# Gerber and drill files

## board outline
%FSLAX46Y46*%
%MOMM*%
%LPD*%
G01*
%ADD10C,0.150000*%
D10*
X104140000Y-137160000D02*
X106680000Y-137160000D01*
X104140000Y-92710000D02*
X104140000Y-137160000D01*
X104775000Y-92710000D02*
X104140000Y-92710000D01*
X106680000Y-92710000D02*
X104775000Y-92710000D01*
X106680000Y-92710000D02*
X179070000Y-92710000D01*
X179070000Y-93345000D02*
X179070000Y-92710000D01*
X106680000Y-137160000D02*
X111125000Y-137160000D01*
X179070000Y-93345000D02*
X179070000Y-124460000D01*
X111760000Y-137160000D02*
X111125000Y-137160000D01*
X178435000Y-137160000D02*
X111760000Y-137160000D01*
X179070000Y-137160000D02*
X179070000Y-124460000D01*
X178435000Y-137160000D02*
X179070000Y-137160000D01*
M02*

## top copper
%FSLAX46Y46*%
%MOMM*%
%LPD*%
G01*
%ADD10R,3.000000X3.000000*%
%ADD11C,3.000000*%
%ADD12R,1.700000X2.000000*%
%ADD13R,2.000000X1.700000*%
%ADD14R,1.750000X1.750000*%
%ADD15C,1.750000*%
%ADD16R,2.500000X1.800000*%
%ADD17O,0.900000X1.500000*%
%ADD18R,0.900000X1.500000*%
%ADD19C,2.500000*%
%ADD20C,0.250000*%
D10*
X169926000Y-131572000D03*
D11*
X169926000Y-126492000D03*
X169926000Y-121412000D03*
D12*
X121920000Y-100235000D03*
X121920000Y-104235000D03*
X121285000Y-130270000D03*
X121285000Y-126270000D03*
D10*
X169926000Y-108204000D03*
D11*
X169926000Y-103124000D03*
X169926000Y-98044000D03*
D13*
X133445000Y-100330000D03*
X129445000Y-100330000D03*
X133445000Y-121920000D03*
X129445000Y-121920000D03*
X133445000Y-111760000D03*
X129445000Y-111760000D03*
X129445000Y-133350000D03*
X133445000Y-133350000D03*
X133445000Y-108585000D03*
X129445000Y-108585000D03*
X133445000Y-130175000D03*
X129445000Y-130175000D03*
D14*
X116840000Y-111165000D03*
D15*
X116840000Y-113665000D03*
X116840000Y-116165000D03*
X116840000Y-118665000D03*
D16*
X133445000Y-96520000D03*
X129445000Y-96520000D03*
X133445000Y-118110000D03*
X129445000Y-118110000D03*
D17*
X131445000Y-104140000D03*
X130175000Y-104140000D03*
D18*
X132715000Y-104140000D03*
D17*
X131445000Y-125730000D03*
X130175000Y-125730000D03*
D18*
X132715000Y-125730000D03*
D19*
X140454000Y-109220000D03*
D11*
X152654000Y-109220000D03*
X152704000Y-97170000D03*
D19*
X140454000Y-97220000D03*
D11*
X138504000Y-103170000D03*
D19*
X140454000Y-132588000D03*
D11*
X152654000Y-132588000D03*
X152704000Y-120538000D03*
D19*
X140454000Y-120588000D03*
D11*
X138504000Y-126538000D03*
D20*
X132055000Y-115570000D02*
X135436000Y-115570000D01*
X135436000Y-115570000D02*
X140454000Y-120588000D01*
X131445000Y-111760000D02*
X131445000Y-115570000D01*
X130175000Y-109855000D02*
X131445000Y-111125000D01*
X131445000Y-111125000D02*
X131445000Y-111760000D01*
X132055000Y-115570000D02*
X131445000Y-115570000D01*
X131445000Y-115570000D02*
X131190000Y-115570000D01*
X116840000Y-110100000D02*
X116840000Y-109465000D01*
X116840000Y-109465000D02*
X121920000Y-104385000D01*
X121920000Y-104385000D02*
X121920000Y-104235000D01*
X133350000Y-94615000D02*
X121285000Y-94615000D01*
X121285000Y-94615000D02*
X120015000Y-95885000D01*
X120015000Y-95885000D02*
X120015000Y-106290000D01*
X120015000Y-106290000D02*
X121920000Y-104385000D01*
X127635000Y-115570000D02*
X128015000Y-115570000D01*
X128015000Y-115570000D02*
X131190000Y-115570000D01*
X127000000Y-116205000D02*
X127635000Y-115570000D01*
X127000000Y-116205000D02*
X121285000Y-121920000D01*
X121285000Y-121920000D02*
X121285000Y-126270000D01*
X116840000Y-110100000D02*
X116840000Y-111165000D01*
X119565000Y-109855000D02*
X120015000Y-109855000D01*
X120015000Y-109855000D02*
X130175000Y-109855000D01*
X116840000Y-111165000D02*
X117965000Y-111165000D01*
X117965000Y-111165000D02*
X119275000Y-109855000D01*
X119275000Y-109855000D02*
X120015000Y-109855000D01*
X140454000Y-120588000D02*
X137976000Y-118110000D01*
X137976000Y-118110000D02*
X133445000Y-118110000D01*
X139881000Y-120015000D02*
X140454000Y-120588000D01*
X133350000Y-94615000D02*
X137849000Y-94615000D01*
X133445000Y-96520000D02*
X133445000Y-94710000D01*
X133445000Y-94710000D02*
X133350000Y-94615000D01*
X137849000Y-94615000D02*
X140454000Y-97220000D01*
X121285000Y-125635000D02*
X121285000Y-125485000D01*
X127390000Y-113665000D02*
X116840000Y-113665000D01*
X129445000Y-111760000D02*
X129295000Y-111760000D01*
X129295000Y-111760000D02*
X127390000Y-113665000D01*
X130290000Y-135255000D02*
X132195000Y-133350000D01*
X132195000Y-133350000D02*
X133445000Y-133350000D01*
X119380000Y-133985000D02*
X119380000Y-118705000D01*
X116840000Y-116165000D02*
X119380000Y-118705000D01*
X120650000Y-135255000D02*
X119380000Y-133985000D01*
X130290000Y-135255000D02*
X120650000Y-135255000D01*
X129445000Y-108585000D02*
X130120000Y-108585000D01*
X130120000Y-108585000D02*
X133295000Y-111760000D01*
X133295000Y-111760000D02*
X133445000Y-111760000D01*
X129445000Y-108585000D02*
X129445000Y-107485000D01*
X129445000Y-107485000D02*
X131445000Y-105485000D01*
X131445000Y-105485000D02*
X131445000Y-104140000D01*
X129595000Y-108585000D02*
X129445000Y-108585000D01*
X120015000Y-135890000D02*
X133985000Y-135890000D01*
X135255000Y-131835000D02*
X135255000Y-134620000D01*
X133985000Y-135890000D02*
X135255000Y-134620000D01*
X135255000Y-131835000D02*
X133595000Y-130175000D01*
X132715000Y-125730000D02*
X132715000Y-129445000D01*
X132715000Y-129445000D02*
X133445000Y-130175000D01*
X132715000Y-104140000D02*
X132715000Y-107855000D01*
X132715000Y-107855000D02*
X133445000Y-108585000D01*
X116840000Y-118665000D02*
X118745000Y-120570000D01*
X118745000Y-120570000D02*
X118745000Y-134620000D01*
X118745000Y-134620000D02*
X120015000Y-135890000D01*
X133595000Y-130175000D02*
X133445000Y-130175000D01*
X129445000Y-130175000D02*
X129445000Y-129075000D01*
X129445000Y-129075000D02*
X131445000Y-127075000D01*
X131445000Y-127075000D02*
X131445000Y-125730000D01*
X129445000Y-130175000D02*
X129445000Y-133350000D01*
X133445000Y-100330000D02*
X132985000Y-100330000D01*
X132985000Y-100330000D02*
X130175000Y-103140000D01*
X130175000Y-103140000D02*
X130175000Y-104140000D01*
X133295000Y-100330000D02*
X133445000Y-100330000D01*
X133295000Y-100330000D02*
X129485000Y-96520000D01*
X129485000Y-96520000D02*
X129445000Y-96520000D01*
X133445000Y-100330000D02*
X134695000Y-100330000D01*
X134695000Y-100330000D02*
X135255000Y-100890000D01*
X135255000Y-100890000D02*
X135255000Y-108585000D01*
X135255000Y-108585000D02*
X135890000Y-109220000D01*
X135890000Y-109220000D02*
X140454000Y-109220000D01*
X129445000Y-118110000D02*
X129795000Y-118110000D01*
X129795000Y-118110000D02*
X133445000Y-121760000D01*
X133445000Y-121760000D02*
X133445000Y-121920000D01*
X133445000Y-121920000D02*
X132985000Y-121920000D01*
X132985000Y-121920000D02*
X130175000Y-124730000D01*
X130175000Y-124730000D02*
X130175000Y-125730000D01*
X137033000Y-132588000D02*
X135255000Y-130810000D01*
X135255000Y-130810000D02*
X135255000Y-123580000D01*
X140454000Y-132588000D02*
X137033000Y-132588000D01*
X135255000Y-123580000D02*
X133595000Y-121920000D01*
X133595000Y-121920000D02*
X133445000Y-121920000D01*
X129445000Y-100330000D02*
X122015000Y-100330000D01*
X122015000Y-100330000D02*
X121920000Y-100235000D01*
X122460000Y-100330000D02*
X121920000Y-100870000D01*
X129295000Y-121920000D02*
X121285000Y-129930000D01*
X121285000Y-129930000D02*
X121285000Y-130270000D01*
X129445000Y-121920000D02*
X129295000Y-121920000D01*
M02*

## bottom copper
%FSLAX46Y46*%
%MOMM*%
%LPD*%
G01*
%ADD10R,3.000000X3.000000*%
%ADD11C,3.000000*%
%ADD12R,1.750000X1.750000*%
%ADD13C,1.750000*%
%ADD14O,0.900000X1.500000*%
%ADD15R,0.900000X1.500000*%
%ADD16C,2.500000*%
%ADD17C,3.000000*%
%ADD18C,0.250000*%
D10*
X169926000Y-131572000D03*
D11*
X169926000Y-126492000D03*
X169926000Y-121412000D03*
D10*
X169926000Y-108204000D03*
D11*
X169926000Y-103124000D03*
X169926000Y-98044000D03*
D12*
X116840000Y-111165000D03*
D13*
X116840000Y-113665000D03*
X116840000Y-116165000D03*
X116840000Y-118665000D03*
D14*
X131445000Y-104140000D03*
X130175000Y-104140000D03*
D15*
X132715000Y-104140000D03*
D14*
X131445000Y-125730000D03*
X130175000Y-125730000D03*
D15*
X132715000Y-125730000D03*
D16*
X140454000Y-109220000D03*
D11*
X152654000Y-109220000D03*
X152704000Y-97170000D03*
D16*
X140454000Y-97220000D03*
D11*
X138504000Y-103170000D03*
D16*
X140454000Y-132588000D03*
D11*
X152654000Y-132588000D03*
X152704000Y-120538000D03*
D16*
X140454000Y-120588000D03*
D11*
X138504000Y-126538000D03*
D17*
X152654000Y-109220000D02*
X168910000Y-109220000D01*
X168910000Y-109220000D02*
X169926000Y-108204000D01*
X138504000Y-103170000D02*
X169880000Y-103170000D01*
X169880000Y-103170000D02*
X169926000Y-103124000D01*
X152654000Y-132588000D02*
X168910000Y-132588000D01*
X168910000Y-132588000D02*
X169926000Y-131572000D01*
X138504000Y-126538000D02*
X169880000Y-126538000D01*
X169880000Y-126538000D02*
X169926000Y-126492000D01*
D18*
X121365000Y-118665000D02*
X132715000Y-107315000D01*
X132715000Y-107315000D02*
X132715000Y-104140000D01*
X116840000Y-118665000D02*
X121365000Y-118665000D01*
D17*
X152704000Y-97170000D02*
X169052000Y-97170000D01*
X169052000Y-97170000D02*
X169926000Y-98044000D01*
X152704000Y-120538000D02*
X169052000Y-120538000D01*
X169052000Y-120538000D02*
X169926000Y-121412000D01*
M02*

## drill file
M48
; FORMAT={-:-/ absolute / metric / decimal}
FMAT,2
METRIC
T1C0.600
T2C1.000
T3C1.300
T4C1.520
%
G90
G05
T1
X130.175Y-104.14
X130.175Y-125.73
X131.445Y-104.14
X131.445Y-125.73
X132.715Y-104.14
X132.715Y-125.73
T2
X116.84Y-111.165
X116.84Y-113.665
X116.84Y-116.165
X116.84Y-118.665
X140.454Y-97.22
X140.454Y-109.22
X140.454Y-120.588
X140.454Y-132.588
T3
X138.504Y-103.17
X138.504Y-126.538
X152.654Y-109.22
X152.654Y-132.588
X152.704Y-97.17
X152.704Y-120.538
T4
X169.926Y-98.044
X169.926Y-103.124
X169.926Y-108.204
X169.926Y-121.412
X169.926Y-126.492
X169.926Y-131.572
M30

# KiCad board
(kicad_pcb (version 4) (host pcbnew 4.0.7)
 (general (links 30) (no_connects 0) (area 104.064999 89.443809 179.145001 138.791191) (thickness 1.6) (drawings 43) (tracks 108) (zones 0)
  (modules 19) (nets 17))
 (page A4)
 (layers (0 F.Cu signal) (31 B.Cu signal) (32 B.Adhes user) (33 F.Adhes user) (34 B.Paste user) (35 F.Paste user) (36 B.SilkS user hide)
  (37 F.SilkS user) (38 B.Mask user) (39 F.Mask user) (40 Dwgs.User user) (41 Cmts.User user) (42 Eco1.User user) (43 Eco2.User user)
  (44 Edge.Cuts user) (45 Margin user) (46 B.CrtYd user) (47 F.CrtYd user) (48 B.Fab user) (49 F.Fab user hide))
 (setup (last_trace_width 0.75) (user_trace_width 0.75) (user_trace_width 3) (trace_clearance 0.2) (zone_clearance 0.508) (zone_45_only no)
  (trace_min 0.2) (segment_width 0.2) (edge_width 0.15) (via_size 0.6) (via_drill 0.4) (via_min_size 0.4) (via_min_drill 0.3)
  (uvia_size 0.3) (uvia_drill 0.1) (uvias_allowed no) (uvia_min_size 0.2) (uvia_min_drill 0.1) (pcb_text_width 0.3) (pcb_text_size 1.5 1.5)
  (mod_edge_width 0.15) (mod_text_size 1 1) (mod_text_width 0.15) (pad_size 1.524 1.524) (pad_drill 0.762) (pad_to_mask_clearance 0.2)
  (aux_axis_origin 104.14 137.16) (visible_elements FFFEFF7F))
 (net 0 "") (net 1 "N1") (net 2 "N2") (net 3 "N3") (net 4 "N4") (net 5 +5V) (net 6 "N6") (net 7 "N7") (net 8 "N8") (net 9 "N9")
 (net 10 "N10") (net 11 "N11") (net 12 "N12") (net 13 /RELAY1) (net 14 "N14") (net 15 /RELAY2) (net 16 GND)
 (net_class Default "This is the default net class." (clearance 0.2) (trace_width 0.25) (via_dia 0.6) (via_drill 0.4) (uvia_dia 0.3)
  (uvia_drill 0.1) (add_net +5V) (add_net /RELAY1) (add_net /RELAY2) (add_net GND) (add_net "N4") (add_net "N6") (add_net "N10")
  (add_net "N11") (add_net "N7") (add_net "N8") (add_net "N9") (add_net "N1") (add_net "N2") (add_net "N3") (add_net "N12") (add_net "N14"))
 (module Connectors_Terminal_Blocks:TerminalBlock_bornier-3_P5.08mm (layer F.Cu) (at 169.926 131.572 90)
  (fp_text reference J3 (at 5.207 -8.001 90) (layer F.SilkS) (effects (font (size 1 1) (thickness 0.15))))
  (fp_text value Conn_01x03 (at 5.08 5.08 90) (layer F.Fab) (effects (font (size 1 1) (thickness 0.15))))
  (pad 1 thru_hole rect (at 0 0 90) (size 3 3) (drill 1.52) (layers *.Cu *.Mask) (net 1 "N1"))
  (pad 2 thru_hole circle (at 5.08 0 90) (size 3 3) (drill 1.52) (layers *.Cu *.Mask) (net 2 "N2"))
  (pad 3 thru_hole circle (at 10.16 0 90) (size 3 3) (drill 1.52) (layers *.Cu *.Mask) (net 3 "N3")))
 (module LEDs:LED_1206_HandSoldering (layer F.Cu) (at 121.92 102.235 270)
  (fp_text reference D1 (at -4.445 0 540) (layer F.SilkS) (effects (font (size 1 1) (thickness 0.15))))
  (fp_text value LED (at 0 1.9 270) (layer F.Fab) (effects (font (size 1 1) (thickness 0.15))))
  (pad 1 smd rect (at -2 0 270) (size 2 1.7) (layers F.Cu F.Paste F.Mask) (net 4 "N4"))
  (pad 2 smd rect (at 2 0 270) (size 2 1.7) (layers F.Cu F.Paste F.Mask) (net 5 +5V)))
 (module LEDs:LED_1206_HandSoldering (layer F.Cu) (at 121.285 128.27 90)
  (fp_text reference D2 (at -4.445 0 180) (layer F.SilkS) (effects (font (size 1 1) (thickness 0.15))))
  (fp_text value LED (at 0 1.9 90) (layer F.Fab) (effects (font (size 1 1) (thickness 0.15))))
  (pad 1 smd rect (at -2 0 90) (size 2 1.7) (layers F.Cu F.Paste F.Mask) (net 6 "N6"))
  (pad 2 smd rect (at 2 0 90) (size 2 1.7) (layers F.Cu F.Paste F.Mask) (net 5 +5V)))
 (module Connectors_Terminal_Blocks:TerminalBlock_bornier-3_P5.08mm (layer F.Cu) (at 169.926 108.204 90)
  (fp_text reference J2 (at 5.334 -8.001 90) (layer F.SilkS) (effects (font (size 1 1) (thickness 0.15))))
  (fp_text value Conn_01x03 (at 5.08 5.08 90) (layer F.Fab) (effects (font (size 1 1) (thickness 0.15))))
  (pad 1 thru_hole rect (at 0 0 90) (size 3 3) (drill 1.52) (layers *.Cu *.Mask) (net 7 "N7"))
  (pad 2 thru_hole circle (at 5.08 0 90) (size 3 3) (drill 1.52) (layers *.Cu *.Mask) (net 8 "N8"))
  (pad 3 thru_hole circle (at 10.16 0 90) (size 3 3) (drill 1.52) (layers *.Cu *.Mask) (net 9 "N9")))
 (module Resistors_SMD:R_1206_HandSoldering (layer F.Cu) (at 131.445 100.33 180)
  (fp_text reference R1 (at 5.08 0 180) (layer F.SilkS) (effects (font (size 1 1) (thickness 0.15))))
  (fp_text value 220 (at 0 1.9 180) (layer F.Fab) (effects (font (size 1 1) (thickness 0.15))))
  (pad 1 smd rect (at -2 0 180) (size 2 1.7) (layers F.Cu F.Paste F.Mask) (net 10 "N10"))
  (pad 2 smd rect (at 2 0 180) (size 2 1.7) (layers F.Cu F.Paste F.Mask) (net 4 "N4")))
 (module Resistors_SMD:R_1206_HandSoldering (layer F.Cu) (at 131.445 121.92 180)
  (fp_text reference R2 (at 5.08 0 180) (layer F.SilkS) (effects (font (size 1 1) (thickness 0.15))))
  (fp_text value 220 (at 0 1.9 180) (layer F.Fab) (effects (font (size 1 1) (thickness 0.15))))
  (pad 1 smd rect (at -2 0 180) (size 2 1.7) (layers F.Cu F.Paste F.Mask) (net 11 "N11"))
  (pad 2 smd rect (at 2 0 180) (size 2 1.7) (layers F.Cu F.Paste F.Mask) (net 6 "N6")))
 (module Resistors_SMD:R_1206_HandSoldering (layer F.Cu) (at 131.445 111.76 180)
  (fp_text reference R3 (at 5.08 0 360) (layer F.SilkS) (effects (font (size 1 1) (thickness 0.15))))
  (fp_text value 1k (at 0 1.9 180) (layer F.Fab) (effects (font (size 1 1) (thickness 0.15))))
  (pad 1 smd rect (at -2 0 180) (size 2 1.7) (layers F.Cu F.Paste F.Mask) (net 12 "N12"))
  (pad 2 smd rect (at 2 0 180) (size 2 1.7) (layers F.Cu F.Paste F.Mask) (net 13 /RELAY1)))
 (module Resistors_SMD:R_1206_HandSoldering (layer F.Cu) (at 131.445 133.35)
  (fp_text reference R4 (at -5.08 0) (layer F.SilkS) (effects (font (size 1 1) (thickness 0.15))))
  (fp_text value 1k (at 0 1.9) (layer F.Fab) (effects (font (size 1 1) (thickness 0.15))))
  (pad 1 smd rect (at -2 0) (size 2 1.7) (layers F.Cu F.Paste F.Mask) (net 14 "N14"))
  (pad 2 smd rect (at 2 0) (size 2 1.7) (layers F.Cu F.Paste F.Mask) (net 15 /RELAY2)))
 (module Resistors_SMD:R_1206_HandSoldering (layer F.Cu) (at 131.445 108.585 180)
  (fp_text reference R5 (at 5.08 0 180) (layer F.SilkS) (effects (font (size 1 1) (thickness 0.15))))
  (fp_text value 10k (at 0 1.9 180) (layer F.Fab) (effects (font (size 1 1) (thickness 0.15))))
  (pad 1 smd rect (at -2 0 180) (size 2 1.7) (layers F.Cu F.Paste F.Mask) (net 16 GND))
  (pad 2 smd rect (at 2 0 180) (size 2 1.7) (layers F.Cu F.Paste F.Mask) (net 12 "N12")))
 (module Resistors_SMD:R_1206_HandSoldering (layer F.Cu) (at 131.445 130.175 180)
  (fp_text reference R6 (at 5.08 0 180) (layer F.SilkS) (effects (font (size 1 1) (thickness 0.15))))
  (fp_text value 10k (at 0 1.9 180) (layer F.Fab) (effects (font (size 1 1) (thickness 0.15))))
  (pad 1 smd rect (at -2 0 180) (size 2 1.7) (layers F.Cu F.Paste F.Mask) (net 16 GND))
  (pad 2 smd rect (at 2 0 180) (size 2 1.7) (layers F.Cu F.Paste F.Mask) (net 14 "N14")))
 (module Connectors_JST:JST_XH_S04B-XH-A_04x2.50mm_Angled (layer F.Cu) (at 116.84 111.165 270)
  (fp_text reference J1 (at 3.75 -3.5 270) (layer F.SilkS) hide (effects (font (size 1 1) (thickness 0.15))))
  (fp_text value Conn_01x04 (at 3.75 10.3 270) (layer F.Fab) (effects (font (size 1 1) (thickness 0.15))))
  (pad 1 thru_hole rect (at 0 0 270) (size 1.75 1.75) (drill 1) (layers *.Cu *.Mask F.SilkS) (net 5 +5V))
  (pad 2 thru_hole circle (at 2.5 0 270) (size 1.75 1.75) (drill 1) (layers *.Cu *.Mask F.SilkS) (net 13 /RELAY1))
  (pad 3 thru_hole circle (at 5 0 270) (size 1.75 1.75) (drill 1) (layers *.Cu *.Mask F.SilkS) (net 15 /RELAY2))
  (pad 4 thru_hole circle (at 7.5 0 270) (size 1.75 1.75) (drill 1) (layers *.Cu *.Mask F.SilkS) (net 16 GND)))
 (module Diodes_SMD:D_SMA (layer F.Cu) (at 131.445 96.52 180)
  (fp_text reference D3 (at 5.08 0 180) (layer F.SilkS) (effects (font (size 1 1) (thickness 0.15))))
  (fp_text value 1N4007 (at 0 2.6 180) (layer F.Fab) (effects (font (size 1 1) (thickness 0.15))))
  (pad 1 smd rect (at -2 0 180) (size 2.5 1.8) (layers F.Cu F.Paste F.Mask) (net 5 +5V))
  (pad 2 smd rect (at 2 0 180) (size 2.5 1.8) (layers F.Cu F.Paste F.Mask) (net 10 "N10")))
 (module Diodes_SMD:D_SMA (layer F.Cu) (at 131.445 118.11 180)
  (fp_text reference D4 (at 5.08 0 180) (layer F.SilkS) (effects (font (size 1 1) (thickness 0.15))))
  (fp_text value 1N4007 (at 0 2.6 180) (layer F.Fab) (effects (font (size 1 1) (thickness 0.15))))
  (pad 1 smd rect (at -2 0 180) (size 2.5 1.8) (layers F.Cu F.Paste F.Mask) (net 5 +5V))
  (pad 2 smd rect (at 2 0 180) (size 2.5 1.8) (layers F.Cu F.Paste F.Mask) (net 11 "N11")))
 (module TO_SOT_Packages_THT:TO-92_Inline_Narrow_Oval (layer F.Cu) (at 132.715 104.14 180)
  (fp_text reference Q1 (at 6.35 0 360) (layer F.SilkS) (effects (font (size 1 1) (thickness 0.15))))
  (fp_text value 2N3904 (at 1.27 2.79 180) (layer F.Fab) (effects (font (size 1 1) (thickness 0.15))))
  (pad 2 thru_hole oval (at 1.27 0) (size 0.9 1.5) (drill 0.6) (layers *.Cu *.Mask) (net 12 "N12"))
  (pad 3 thru_hole oval (at 2.54 0) (size 0.9 1.5) (drill 0.6) (layers *.Cu *.Mask) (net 10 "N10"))
  (pad 1 thru_hole rect (at 0 0) (size 0.9 1.5) (drill 0.6) (layers *.Cu *.Mask) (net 16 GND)))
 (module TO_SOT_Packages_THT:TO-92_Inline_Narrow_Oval (layer F.Cu) (at 132.715 125.73 180)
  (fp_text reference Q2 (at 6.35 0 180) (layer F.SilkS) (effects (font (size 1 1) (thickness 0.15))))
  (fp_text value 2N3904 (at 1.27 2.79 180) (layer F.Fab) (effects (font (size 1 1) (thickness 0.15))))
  (pad 2 thru_hole oval (at 1.27 0) (size 0.9 1.5) (drill 0.6) (layers *.Cu *.Mask) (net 14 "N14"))
  (pad 3 thru_hole oval (at 2.54 0) (size 0.9 1.5) (drill 0.6) (layers *.Cu *.Mask) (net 11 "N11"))
  (pad 1 thru_hole rect (at 0 0) (size 0.9 1.5) (drill 0.6) (layers *.Cu *.Mask) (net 16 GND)))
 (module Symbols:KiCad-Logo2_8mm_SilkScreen (layer B.Cu) (at 161.29 126.365 270)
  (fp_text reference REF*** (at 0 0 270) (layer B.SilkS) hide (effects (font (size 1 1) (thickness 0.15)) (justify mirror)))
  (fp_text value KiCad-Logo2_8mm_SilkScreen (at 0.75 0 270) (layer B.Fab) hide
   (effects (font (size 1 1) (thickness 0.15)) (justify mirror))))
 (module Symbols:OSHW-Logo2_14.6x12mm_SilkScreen (layer B.Cu) (at 160.655 102.87 270)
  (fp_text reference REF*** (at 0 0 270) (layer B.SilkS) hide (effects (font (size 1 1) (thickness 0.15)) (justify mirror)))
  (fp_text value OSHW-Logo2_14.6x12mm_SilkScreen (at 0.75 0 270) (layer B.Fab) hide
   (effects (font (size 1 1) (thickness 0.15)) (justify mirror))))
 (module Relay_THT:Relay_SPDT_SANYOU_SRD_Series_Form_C (layer F.Cu) (at 138.504 103.17)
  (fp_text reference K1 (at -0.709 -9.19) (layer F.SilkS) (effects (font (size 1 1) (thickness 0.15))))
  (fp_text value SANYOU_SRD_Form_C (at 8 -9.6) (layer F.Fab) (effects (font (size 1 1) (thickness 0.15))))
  (pad 2 thru_hole circle (at 1.95 6.05 90) (size 2.5 2.5) (drill 1) (layers *.Cu *.Mask) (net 10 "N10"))
  (pad 3 thru_hole circle (at 14.15 6.05 90) (size 3 3) (drill 1.3) (layers *.Cu *.Mask) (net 7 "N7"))
  (pad 4 thru_hole circle (at 14.2 -6 90) (size 3 3) (drill 1.3) (layers *.Cu *.Mask) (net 9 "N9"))
  (pad 5 thru_hole circle (at 1.95 -5.95 90) (size 2.5 2.5) (drill 1) (layers *.Cu *.Mask) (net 5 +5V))
  (pad 1 thru_hole circle (at 0 0 90) (size 3 3) (drill 1.3) (layers *.Cu *.Mask) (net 8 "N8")))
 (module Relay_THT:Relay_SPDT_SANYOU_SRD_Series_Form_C (layer F.Cu) (at 138.504 126.538)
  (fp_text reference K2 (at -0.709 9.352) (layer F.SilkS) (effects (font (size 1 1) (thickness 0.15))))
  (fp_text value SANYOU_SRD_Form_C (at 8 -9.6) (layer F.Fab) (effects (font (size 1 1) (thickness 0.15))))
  (pad 2 thru_hole circle (at 1.95 6.05 90) (size 2.5 2.5) (drill 1) (layers *.Cu *.Mask) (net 11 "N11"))
  (pad 3 thru_hole circle (at 14.15 6.05 90) (size 3 3) (drill 1.3) (layers *.Cu *.Mask) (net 1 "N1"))
  (pad 4 thru_hole circle (at 14.2 -6 90) (size 3 3) (drill 1.3) (layers *.Cu *.Mask) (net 3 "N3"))
  (pad 5 thru_hole circle (at 1.95 -5.95 90) (size 2.5 2.5) (drill 1) (layers *.Cu *.Mask) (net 5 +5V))
  (pad 1 thru_hole circle (at 0 0 90) (size 3 3) (drill 1.3) (layers *.Cu *.Mask) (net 2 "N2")))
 (gr_line (start 104.14 137.16) (end 106.68 137.16) (layer Edge.Cuts) (width 0.15))
 (gr_line (start 104.14 92.71) (end 104.14 137.16) (layer Edge.Cuts) (width 0.15))
 (gr_line (start 104.775 92.71) (end 104.14 92.71) (layer Edge.Cuts) (width 0.15))
 (gr_line (start 106.68 92.71) (end 104.775 92.71) (layer Edge.Cuts) (width 0.15))
 (gr_line (start 106.68 92.71) (end 179.07 92.71) (layer Edge.Cuts) (width 0.15))
 (gr_line (start 179.07 93.345) (end 179.07 92.71) (layer Edge.Cuts) (width 0.15))
 (gr_line (start 106.68 137.16) (end 111.125 137.16) (layer Edge.Cuts) (width 0.15))
 (gr_line (start 179.07 93.345) (end 179.07 124.46) (layer Edge.Cuts) (width 0.15))
 (gr_line (start 111.76 137.16) (end 111.125 137.16) (layer Edge.Cuts) (width 0.15))
 (gr_line (start 178.435 137.16) (end 111.76 137.16) (layer Edge.Cuts) (width 0.15))
 (gr_line (start 179.07 137.16) (end 179.07 124.46) (layer Edge.Cuts) (width 0.15))
 (gr_line (start 178.435 137.16) (end 179.07 137.16) (layer Edge.Cuts) (width 0.15))
 (segment (start 132.055 115.57) (end 135.436 115.57) (width 0.25) (layer F.Cu) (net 5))
 (segment (start 135.436 115.57) (end 140.454 120.588) (width 0.25) (layer F.Cu) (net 5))
 (segment (start 131.445 111.76) (end 131.445 115.57) (width 0.25) (layer F.Cu) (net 5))
 (segment (start 130.175 109.855) (end 131.445 111.125) (width 0.25) (layer F.Cu) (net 5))
 (segment (start 131.445 111.125) (end 131.445 111.76) (width 0.25) (layer F.Cu) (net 5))
 (segment (start 132.055 115.57) (end 131.445 115.57) (width 0.25) (layer F.Cu) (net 5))
 (segment (start 131.445 115.57) (end 131.19 115.57) (width 0.25) (layer F.Cu) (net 5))
 (segment (start 116.84 110.1) (end 116.84 109.465) (width 0.25) (layer F.Cu) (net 5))
 (segment (start 116.84 109.465) (end 121.92 104.385) (width 0.25) (layer F.Cu) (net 5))
 (segment (start 121.92 104.385) (end 121.92 104.235) (width 0.25) (layer F.Cu) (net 5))
 (segment (start 133.35 94.615) (end 121.285 94.615) (width 0.25) (layer F.Cu) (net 5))
 (segment (start 121.285 94.615) (end 120.015 95.885) (width 0.25) (layer F.Cu) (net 5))
 (segment (start 120.015 95.885) (end 120.015 106.29) (width 0.25) (layer F.Cu) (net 5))
 (segment (start 120.015 106.29) (end 121.92 104.385) (width 0.25) (layer F.Cu) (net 5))
 (segment (start 127.635 115.57) (end 128.015 115.57) (width 0.25) (layer F.Cu) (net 5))
 (segment (start 128.015 115.57) (end 131.19 115.57) (width 0.25) (layer F.Cu) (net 5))
 (segment (start 127 116.205) (end 127.635 115.57) (width 0.25) (layer F.Cu) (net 5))
 (segment (start 127 116.205) (end 121.285 121.92) (width 0.25) (layer F.Cu) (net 5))
 (segment (start 121.285 121.92) (end 121.285 126.27) (width 0.25) (layer F.Cu) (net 5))
 (segment (start 116.84 110.1) (end 116.84 111.165) (width 0.25) (layer F.Cu) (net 5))
 (segment (start 119.565 109.855) (end 120.015 109.855) (width 0.25) (layer F.Cu) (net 5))
 (segment (start 120.015 109.855) (end 130.175 109.855) (width 0.25) (layer F.Cu) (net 5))
 (segment (start 116.84 111.165) (end 117.965 111.165) (width 0.25) (layer F.Cu) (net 5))
 (segment (start 117.965 111.165) (end 119.275 109.855) (width 0.25) (layer F.Cu) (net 5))
 (segment (start 119.275 109.855) (end 120.015 109.855) (width 0.25) (layer F.Cu) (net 5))
 (segment (start 140.454 120.588) (end 137.976 118.11) (width 0.25) (layer F.Cu) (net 5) (status 10))
 (segment (start 137.976 118.11) (end 133.445 118.11) (width 0.25) (layer F.Cu) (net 5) (status 20))
 (segment (start 139.881 120.015) (end 140.454 120.588) (width 0.25) (layer F.Cu) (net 5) (status 30))
 (segment (start 133.35 94.615) (end 137.849 94.615) (width 0.25) (layer F.Cu) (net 5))
 (segment (start 133.445 96.52) (end 133.445 94.71) (width 0.25) (layer F.Cu) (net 5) (status 10))
 (segment (start 133.445 94.71) (end 133.35 94.615) (width 0.25) (layer F.Cu) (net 5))
 (segment (start 137.849 94.615) (end 140.454 97.22) (width 0.25) (layer F.Cu) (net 5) (status 20))
 (segment (start 121.285 125.635) (end 121.285 125.485) (width 0.25) (layer F.Cu) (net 5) (status 30))
 (segment (start 127.39 113.665) (end 116.84 113.665) (width 0.25) (layer F.Cu) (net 13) (status 20))
 (segment (start 129.445 111.76) (end 129.295 111.76) (width 0.25) (layer F.Cu) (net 13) (status 30))
 (segment (start 129.295 111.76) (end 127.39 113.665) (width 0.25) (layer F.Cu) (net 13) (status 10))
 (segment (start 130.29 135.255) (end 132.195 133.35) (width 0.25) (layer F.Cu) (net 15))
 (segment (start 132.195 133.35) (end 133.445 133.35) (width 0.25) (layer F.Cu) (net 15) (status 20))
 (segment (start 119.38 133.985) (end 119.38 118.705) (width 0.25) (layer F.Cu) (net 15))
 (segment (start 116.84 116.165) (end 119.38 118.705) (width 0.25) (layer F.Cu) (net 15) (status 10))
 (segment (start 120.65 135.255) (end 119.38 133.985) (width 0.25) (layer F.Cu) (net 15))
 (segment (start 130.29 135.255) (end 120.65 135.255) (width 0.25) (layer F.Cu) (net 15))
 (segment (start 152.654 109.22) (end 168.91 109.22) (width 3) (layer B.Cu) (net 7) (status 30))
 (segment (start 168.91 109.22) (end 169.926 108.204) (width 3) (layer B.Cu) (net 7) (status 30))
 (segment (start 138.504 103.17) (end 169.88 103.17) (width 3) (layer B.Cu) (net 8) (status 30))
 (segment (start 169.88 103.17) (end 169.926 103.124) (width 3) (layer B.Cu) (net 8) (status 30))
 (segment (start 152.654 132.588) (end 168.91 132.588) (width 3) (layer B.Cu) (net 1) (status 30))
 (segment (start 168.91 132.588) (end 169.926 131.572) (width 3) (layer B.Cu) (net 1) (status 30))
 (segment (start 138.504 126.538) (end 169.88 126.538) (width 3) (layer B.Cu) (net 2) (status 30))
 (segment (start 169.88 126.538) (end 169.926 126.492) (width 3) (layer B.Cu) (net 2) (status 30))
 (segment (start 129.445 108.585) (end 130.12 108.585) (width 0.25) (layer F.Cu) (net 12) (status 30))
 (segment (start 130.12 108.585) (end 133.295 111.76) (width 0.25) (layer F.Cu) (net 12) (status 30))
 (segment (start 133.295 111.76) (end 133.445 111.76) (width 0.25) (layer F.Cu) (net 12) (status 30))
 (segment (start 129.445 108.585) (end 129.445 107.485) (width 0.25) (layer F.Cu) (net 12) (status 10))
 (segment (start 129.445 107.485) (end 131.445 105.485) (width 0.25) (layer F.Cu) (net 12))
 (segment (start 131.445 105.485) (end 131.445 104.14) (width 0.25) (layer F.Cu) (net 12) (status 20))
 (segment (start 129.595 108.585) (end 129.445 108.585) (width 0.25) (layer F.Cu) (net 12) (status 30))
 (segment (start 120.015 135.89) (end 133.985 135.89) (width 0.25) (layer F.Cu) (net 16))
 (segment (start 135.255 131.835) (end 135.255 134.62) (width 0.25) (layer F.Cu) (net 16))
 (segment (start 133.985 135.89) (end 135.255 134.62) (width 0.25) (layer F.Cu) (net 16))
 (segment (start 135.255 131.835) (end 133.595 130.175) (width 0.25) (layer F.Cu) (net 16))
 (segment (start 121.365 118.665) (end 132.715 107.315) (width 0.25) (layer B.Cu) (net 16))
 (segment (start 132.715 107.315) (end 132.715 104.14) (width 0.25) (layer B.Cu) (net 16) (status 20))
 (segment (start 116.84 118.665) (end 121.365 118.665) (width 0.25) (layer B.Cu) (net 16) (status 10))
 (segment (start 132.715 125.73) (end 132.715 129.445) (width 0.25) (layer F.Cu) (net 16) (status 30))
 (segment (start 132.715 129.445) (end 133.445 130.175) (width 0.25) (layer F.Cu) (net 16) (status 30))
 (segment (start 132.715 104.14) (end 132.715 107.855) (width 0.25) (layer F.Cu) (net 16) (status 30))
 (segment (start 132.715 107.855) (end 133.445 108.585) (width 0.25) (layer F.Cu) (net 16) (status 30))
 (segment (start 116.84 118.665) (end 118.745 120.57) (width 0.25) (layer F.Cu) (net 16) (status 10))
 (segment (start 118.745 120.57) (end 118.745 134.62) (width 0.25) (layer F.Cu) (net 16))
 (segment (start 118.745 134.62) (end 120.015 135.89) (width 0.25) (layer F.Cu) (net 16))
 (segment (start 133.595 130.175) (end 133.445 130.175) (width 0.25) (layer F.Cu) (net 16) (status 30))
 (segment (start 129.445 130.175) (end 129.445 129.075) (width 0.25) (layer F.Cu) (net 14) (status 10))
 (segment (start 129.445 129.075) (end 131.445 127.075) (width 0.25) (layer F.Cu) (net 14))
 (segment (start 131.445 127.075) (end 131.445 125.73) (width 0.25) (layer F.Cu) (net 14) (status 20))
 (segment (start 129.445 130.175) (end 129.445 133.35) (width 0.25) (layer F.Cu) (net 14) (status 30))
 (segment (start 152.704 97.17) (end 169.052 97.17) (width 3) (layer B.Cu) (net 9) (status 30))
 (segment (start 169.052 97.17) (end 169.926 98.044) (width 3) (layer B.Cu) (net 9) (status 30))
 (segment (start 152.704 120.538) (end 169.052 120.538) (width 3) (layer B.Cu) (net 3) (status 30))
 (segment (start 169.052 120.538) (end 169.926 121.412) (width 3) (layer B.Cu) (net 3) (status 30))
 (segment (start 133.445 100.33) (end 132.985 100.33) (width 0.25) (layer F.Cu) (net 10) (status 30))
 (segment (start 132.985 100.33) (end 130.175 103.14) (width 0.25) (layer F.Cu) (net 10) (status 10))
 (segment (start 130.175 103.14) (end 130.175 104.14) (width 0.25) (layer F.Cu) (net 10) (status 20))
 (segment (start 133.295 100.33) (end 133.445 100.33) (width 0.25) (layer F.Cu) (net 10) (status 30))
 (segment (start 133.295 100.33) (end 129.485 96.52) (width 0.25) (layer F.Cu) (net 10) (status 30))
 (segment (start 129.485 96.52) (end 129.445 96.52) (width 0.25) (layer F.Cu) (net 10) (status 30))
 (segment (start 133.445 100.33) (end 134.695 100.33) (width 0.25) (layer F.Cu) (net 10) (status 10))
 (segment (start 134.695 100.33) (end 135.255 100.89) (width 0.25) (layer F.Cu) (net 10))
 (segment (start 135.255 100.89) (end 135.255 108.585) (width 0.25) (layer F.Cu) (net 10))
 (segment (start 135.255 108.585) (end 135.89 109.22) (width 0.25) (layer F.Cu) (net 10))
 (segment (start 135.89 109.22) (end 140.454 109.22) (width 0.25) (layer F.Cu) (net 10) (status 20))
 (segment (start 129.445 118.11) (end 129.795 118.11) (width 0.25) (layer F.Cu) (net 11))
 (segment (start 129.795 118.11) (end 133.445 121.76) (width 0.25) (layer F.Cu) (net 11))
 (segment (start 133.445 121.76) (end 133.445 121.92) (width 0.25) (layer F.Cu) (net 11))
 (segment (start 133.445 121.92) (end 132.985 121.92) (width 0.25) (layer F.Cu) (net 11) (status 30))
 (segment (start 132.985 121.92) (end 130.175 124.73) (width 0.25) (layer F.Cu) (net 11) (status 10))
 (segment (start 130.175 124.73) (end 130.175 125.73) (width 0.25) (layer F.Cu) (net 11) (status 20))
 (segment (start 137.033 132.588) (end 135.255 130.81) (width 0.25) (layer F.Cu) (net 11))
 (segment (start 135.255 130.81) (end 135.255 123.58) (width 0.25) (layer F.Cu) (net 11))
 (segment (start 140.454 132.588) (end 137.033 132.588) (width 0.25) (layer F.Cu) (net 11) (status 10))
 (segment (start 135.255 123.58) (end 133.595 121.92) (width 0.25) (layer F.Cu) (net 11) (status 20))
 (segment (start 133.595 121.92) (end 133.445 121.92) (width 0.25) (layer F.Cu) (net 11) (status 30))
 (segment (start 129.445 100.33) (end 122.015 100.33) (width 0.25) (layer F.Cu) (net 4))
 (segment (start 122.015 100.33) (end 121.92 100.235) (width 0.25) (layer F.Cu) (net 4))
 (segment (start 122.46 100.33) (end 121.92 100.87) (width 0.25) (layer F.Cu) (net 4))
 (segment (start 129.295 121.92) (end 121.285 129.93) (width 0.25) (layer F.Cu) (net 6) (status 30))
 (segment (start 121.285 129.93) (end 121.285 130.27) (width 0.25) (layer F.Cu) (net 6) (status 30))
 (segment (start 129.445 121.92) (end 129.295 121.92) (width 0.25) (layer F.Cu) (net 6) (status 30)))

